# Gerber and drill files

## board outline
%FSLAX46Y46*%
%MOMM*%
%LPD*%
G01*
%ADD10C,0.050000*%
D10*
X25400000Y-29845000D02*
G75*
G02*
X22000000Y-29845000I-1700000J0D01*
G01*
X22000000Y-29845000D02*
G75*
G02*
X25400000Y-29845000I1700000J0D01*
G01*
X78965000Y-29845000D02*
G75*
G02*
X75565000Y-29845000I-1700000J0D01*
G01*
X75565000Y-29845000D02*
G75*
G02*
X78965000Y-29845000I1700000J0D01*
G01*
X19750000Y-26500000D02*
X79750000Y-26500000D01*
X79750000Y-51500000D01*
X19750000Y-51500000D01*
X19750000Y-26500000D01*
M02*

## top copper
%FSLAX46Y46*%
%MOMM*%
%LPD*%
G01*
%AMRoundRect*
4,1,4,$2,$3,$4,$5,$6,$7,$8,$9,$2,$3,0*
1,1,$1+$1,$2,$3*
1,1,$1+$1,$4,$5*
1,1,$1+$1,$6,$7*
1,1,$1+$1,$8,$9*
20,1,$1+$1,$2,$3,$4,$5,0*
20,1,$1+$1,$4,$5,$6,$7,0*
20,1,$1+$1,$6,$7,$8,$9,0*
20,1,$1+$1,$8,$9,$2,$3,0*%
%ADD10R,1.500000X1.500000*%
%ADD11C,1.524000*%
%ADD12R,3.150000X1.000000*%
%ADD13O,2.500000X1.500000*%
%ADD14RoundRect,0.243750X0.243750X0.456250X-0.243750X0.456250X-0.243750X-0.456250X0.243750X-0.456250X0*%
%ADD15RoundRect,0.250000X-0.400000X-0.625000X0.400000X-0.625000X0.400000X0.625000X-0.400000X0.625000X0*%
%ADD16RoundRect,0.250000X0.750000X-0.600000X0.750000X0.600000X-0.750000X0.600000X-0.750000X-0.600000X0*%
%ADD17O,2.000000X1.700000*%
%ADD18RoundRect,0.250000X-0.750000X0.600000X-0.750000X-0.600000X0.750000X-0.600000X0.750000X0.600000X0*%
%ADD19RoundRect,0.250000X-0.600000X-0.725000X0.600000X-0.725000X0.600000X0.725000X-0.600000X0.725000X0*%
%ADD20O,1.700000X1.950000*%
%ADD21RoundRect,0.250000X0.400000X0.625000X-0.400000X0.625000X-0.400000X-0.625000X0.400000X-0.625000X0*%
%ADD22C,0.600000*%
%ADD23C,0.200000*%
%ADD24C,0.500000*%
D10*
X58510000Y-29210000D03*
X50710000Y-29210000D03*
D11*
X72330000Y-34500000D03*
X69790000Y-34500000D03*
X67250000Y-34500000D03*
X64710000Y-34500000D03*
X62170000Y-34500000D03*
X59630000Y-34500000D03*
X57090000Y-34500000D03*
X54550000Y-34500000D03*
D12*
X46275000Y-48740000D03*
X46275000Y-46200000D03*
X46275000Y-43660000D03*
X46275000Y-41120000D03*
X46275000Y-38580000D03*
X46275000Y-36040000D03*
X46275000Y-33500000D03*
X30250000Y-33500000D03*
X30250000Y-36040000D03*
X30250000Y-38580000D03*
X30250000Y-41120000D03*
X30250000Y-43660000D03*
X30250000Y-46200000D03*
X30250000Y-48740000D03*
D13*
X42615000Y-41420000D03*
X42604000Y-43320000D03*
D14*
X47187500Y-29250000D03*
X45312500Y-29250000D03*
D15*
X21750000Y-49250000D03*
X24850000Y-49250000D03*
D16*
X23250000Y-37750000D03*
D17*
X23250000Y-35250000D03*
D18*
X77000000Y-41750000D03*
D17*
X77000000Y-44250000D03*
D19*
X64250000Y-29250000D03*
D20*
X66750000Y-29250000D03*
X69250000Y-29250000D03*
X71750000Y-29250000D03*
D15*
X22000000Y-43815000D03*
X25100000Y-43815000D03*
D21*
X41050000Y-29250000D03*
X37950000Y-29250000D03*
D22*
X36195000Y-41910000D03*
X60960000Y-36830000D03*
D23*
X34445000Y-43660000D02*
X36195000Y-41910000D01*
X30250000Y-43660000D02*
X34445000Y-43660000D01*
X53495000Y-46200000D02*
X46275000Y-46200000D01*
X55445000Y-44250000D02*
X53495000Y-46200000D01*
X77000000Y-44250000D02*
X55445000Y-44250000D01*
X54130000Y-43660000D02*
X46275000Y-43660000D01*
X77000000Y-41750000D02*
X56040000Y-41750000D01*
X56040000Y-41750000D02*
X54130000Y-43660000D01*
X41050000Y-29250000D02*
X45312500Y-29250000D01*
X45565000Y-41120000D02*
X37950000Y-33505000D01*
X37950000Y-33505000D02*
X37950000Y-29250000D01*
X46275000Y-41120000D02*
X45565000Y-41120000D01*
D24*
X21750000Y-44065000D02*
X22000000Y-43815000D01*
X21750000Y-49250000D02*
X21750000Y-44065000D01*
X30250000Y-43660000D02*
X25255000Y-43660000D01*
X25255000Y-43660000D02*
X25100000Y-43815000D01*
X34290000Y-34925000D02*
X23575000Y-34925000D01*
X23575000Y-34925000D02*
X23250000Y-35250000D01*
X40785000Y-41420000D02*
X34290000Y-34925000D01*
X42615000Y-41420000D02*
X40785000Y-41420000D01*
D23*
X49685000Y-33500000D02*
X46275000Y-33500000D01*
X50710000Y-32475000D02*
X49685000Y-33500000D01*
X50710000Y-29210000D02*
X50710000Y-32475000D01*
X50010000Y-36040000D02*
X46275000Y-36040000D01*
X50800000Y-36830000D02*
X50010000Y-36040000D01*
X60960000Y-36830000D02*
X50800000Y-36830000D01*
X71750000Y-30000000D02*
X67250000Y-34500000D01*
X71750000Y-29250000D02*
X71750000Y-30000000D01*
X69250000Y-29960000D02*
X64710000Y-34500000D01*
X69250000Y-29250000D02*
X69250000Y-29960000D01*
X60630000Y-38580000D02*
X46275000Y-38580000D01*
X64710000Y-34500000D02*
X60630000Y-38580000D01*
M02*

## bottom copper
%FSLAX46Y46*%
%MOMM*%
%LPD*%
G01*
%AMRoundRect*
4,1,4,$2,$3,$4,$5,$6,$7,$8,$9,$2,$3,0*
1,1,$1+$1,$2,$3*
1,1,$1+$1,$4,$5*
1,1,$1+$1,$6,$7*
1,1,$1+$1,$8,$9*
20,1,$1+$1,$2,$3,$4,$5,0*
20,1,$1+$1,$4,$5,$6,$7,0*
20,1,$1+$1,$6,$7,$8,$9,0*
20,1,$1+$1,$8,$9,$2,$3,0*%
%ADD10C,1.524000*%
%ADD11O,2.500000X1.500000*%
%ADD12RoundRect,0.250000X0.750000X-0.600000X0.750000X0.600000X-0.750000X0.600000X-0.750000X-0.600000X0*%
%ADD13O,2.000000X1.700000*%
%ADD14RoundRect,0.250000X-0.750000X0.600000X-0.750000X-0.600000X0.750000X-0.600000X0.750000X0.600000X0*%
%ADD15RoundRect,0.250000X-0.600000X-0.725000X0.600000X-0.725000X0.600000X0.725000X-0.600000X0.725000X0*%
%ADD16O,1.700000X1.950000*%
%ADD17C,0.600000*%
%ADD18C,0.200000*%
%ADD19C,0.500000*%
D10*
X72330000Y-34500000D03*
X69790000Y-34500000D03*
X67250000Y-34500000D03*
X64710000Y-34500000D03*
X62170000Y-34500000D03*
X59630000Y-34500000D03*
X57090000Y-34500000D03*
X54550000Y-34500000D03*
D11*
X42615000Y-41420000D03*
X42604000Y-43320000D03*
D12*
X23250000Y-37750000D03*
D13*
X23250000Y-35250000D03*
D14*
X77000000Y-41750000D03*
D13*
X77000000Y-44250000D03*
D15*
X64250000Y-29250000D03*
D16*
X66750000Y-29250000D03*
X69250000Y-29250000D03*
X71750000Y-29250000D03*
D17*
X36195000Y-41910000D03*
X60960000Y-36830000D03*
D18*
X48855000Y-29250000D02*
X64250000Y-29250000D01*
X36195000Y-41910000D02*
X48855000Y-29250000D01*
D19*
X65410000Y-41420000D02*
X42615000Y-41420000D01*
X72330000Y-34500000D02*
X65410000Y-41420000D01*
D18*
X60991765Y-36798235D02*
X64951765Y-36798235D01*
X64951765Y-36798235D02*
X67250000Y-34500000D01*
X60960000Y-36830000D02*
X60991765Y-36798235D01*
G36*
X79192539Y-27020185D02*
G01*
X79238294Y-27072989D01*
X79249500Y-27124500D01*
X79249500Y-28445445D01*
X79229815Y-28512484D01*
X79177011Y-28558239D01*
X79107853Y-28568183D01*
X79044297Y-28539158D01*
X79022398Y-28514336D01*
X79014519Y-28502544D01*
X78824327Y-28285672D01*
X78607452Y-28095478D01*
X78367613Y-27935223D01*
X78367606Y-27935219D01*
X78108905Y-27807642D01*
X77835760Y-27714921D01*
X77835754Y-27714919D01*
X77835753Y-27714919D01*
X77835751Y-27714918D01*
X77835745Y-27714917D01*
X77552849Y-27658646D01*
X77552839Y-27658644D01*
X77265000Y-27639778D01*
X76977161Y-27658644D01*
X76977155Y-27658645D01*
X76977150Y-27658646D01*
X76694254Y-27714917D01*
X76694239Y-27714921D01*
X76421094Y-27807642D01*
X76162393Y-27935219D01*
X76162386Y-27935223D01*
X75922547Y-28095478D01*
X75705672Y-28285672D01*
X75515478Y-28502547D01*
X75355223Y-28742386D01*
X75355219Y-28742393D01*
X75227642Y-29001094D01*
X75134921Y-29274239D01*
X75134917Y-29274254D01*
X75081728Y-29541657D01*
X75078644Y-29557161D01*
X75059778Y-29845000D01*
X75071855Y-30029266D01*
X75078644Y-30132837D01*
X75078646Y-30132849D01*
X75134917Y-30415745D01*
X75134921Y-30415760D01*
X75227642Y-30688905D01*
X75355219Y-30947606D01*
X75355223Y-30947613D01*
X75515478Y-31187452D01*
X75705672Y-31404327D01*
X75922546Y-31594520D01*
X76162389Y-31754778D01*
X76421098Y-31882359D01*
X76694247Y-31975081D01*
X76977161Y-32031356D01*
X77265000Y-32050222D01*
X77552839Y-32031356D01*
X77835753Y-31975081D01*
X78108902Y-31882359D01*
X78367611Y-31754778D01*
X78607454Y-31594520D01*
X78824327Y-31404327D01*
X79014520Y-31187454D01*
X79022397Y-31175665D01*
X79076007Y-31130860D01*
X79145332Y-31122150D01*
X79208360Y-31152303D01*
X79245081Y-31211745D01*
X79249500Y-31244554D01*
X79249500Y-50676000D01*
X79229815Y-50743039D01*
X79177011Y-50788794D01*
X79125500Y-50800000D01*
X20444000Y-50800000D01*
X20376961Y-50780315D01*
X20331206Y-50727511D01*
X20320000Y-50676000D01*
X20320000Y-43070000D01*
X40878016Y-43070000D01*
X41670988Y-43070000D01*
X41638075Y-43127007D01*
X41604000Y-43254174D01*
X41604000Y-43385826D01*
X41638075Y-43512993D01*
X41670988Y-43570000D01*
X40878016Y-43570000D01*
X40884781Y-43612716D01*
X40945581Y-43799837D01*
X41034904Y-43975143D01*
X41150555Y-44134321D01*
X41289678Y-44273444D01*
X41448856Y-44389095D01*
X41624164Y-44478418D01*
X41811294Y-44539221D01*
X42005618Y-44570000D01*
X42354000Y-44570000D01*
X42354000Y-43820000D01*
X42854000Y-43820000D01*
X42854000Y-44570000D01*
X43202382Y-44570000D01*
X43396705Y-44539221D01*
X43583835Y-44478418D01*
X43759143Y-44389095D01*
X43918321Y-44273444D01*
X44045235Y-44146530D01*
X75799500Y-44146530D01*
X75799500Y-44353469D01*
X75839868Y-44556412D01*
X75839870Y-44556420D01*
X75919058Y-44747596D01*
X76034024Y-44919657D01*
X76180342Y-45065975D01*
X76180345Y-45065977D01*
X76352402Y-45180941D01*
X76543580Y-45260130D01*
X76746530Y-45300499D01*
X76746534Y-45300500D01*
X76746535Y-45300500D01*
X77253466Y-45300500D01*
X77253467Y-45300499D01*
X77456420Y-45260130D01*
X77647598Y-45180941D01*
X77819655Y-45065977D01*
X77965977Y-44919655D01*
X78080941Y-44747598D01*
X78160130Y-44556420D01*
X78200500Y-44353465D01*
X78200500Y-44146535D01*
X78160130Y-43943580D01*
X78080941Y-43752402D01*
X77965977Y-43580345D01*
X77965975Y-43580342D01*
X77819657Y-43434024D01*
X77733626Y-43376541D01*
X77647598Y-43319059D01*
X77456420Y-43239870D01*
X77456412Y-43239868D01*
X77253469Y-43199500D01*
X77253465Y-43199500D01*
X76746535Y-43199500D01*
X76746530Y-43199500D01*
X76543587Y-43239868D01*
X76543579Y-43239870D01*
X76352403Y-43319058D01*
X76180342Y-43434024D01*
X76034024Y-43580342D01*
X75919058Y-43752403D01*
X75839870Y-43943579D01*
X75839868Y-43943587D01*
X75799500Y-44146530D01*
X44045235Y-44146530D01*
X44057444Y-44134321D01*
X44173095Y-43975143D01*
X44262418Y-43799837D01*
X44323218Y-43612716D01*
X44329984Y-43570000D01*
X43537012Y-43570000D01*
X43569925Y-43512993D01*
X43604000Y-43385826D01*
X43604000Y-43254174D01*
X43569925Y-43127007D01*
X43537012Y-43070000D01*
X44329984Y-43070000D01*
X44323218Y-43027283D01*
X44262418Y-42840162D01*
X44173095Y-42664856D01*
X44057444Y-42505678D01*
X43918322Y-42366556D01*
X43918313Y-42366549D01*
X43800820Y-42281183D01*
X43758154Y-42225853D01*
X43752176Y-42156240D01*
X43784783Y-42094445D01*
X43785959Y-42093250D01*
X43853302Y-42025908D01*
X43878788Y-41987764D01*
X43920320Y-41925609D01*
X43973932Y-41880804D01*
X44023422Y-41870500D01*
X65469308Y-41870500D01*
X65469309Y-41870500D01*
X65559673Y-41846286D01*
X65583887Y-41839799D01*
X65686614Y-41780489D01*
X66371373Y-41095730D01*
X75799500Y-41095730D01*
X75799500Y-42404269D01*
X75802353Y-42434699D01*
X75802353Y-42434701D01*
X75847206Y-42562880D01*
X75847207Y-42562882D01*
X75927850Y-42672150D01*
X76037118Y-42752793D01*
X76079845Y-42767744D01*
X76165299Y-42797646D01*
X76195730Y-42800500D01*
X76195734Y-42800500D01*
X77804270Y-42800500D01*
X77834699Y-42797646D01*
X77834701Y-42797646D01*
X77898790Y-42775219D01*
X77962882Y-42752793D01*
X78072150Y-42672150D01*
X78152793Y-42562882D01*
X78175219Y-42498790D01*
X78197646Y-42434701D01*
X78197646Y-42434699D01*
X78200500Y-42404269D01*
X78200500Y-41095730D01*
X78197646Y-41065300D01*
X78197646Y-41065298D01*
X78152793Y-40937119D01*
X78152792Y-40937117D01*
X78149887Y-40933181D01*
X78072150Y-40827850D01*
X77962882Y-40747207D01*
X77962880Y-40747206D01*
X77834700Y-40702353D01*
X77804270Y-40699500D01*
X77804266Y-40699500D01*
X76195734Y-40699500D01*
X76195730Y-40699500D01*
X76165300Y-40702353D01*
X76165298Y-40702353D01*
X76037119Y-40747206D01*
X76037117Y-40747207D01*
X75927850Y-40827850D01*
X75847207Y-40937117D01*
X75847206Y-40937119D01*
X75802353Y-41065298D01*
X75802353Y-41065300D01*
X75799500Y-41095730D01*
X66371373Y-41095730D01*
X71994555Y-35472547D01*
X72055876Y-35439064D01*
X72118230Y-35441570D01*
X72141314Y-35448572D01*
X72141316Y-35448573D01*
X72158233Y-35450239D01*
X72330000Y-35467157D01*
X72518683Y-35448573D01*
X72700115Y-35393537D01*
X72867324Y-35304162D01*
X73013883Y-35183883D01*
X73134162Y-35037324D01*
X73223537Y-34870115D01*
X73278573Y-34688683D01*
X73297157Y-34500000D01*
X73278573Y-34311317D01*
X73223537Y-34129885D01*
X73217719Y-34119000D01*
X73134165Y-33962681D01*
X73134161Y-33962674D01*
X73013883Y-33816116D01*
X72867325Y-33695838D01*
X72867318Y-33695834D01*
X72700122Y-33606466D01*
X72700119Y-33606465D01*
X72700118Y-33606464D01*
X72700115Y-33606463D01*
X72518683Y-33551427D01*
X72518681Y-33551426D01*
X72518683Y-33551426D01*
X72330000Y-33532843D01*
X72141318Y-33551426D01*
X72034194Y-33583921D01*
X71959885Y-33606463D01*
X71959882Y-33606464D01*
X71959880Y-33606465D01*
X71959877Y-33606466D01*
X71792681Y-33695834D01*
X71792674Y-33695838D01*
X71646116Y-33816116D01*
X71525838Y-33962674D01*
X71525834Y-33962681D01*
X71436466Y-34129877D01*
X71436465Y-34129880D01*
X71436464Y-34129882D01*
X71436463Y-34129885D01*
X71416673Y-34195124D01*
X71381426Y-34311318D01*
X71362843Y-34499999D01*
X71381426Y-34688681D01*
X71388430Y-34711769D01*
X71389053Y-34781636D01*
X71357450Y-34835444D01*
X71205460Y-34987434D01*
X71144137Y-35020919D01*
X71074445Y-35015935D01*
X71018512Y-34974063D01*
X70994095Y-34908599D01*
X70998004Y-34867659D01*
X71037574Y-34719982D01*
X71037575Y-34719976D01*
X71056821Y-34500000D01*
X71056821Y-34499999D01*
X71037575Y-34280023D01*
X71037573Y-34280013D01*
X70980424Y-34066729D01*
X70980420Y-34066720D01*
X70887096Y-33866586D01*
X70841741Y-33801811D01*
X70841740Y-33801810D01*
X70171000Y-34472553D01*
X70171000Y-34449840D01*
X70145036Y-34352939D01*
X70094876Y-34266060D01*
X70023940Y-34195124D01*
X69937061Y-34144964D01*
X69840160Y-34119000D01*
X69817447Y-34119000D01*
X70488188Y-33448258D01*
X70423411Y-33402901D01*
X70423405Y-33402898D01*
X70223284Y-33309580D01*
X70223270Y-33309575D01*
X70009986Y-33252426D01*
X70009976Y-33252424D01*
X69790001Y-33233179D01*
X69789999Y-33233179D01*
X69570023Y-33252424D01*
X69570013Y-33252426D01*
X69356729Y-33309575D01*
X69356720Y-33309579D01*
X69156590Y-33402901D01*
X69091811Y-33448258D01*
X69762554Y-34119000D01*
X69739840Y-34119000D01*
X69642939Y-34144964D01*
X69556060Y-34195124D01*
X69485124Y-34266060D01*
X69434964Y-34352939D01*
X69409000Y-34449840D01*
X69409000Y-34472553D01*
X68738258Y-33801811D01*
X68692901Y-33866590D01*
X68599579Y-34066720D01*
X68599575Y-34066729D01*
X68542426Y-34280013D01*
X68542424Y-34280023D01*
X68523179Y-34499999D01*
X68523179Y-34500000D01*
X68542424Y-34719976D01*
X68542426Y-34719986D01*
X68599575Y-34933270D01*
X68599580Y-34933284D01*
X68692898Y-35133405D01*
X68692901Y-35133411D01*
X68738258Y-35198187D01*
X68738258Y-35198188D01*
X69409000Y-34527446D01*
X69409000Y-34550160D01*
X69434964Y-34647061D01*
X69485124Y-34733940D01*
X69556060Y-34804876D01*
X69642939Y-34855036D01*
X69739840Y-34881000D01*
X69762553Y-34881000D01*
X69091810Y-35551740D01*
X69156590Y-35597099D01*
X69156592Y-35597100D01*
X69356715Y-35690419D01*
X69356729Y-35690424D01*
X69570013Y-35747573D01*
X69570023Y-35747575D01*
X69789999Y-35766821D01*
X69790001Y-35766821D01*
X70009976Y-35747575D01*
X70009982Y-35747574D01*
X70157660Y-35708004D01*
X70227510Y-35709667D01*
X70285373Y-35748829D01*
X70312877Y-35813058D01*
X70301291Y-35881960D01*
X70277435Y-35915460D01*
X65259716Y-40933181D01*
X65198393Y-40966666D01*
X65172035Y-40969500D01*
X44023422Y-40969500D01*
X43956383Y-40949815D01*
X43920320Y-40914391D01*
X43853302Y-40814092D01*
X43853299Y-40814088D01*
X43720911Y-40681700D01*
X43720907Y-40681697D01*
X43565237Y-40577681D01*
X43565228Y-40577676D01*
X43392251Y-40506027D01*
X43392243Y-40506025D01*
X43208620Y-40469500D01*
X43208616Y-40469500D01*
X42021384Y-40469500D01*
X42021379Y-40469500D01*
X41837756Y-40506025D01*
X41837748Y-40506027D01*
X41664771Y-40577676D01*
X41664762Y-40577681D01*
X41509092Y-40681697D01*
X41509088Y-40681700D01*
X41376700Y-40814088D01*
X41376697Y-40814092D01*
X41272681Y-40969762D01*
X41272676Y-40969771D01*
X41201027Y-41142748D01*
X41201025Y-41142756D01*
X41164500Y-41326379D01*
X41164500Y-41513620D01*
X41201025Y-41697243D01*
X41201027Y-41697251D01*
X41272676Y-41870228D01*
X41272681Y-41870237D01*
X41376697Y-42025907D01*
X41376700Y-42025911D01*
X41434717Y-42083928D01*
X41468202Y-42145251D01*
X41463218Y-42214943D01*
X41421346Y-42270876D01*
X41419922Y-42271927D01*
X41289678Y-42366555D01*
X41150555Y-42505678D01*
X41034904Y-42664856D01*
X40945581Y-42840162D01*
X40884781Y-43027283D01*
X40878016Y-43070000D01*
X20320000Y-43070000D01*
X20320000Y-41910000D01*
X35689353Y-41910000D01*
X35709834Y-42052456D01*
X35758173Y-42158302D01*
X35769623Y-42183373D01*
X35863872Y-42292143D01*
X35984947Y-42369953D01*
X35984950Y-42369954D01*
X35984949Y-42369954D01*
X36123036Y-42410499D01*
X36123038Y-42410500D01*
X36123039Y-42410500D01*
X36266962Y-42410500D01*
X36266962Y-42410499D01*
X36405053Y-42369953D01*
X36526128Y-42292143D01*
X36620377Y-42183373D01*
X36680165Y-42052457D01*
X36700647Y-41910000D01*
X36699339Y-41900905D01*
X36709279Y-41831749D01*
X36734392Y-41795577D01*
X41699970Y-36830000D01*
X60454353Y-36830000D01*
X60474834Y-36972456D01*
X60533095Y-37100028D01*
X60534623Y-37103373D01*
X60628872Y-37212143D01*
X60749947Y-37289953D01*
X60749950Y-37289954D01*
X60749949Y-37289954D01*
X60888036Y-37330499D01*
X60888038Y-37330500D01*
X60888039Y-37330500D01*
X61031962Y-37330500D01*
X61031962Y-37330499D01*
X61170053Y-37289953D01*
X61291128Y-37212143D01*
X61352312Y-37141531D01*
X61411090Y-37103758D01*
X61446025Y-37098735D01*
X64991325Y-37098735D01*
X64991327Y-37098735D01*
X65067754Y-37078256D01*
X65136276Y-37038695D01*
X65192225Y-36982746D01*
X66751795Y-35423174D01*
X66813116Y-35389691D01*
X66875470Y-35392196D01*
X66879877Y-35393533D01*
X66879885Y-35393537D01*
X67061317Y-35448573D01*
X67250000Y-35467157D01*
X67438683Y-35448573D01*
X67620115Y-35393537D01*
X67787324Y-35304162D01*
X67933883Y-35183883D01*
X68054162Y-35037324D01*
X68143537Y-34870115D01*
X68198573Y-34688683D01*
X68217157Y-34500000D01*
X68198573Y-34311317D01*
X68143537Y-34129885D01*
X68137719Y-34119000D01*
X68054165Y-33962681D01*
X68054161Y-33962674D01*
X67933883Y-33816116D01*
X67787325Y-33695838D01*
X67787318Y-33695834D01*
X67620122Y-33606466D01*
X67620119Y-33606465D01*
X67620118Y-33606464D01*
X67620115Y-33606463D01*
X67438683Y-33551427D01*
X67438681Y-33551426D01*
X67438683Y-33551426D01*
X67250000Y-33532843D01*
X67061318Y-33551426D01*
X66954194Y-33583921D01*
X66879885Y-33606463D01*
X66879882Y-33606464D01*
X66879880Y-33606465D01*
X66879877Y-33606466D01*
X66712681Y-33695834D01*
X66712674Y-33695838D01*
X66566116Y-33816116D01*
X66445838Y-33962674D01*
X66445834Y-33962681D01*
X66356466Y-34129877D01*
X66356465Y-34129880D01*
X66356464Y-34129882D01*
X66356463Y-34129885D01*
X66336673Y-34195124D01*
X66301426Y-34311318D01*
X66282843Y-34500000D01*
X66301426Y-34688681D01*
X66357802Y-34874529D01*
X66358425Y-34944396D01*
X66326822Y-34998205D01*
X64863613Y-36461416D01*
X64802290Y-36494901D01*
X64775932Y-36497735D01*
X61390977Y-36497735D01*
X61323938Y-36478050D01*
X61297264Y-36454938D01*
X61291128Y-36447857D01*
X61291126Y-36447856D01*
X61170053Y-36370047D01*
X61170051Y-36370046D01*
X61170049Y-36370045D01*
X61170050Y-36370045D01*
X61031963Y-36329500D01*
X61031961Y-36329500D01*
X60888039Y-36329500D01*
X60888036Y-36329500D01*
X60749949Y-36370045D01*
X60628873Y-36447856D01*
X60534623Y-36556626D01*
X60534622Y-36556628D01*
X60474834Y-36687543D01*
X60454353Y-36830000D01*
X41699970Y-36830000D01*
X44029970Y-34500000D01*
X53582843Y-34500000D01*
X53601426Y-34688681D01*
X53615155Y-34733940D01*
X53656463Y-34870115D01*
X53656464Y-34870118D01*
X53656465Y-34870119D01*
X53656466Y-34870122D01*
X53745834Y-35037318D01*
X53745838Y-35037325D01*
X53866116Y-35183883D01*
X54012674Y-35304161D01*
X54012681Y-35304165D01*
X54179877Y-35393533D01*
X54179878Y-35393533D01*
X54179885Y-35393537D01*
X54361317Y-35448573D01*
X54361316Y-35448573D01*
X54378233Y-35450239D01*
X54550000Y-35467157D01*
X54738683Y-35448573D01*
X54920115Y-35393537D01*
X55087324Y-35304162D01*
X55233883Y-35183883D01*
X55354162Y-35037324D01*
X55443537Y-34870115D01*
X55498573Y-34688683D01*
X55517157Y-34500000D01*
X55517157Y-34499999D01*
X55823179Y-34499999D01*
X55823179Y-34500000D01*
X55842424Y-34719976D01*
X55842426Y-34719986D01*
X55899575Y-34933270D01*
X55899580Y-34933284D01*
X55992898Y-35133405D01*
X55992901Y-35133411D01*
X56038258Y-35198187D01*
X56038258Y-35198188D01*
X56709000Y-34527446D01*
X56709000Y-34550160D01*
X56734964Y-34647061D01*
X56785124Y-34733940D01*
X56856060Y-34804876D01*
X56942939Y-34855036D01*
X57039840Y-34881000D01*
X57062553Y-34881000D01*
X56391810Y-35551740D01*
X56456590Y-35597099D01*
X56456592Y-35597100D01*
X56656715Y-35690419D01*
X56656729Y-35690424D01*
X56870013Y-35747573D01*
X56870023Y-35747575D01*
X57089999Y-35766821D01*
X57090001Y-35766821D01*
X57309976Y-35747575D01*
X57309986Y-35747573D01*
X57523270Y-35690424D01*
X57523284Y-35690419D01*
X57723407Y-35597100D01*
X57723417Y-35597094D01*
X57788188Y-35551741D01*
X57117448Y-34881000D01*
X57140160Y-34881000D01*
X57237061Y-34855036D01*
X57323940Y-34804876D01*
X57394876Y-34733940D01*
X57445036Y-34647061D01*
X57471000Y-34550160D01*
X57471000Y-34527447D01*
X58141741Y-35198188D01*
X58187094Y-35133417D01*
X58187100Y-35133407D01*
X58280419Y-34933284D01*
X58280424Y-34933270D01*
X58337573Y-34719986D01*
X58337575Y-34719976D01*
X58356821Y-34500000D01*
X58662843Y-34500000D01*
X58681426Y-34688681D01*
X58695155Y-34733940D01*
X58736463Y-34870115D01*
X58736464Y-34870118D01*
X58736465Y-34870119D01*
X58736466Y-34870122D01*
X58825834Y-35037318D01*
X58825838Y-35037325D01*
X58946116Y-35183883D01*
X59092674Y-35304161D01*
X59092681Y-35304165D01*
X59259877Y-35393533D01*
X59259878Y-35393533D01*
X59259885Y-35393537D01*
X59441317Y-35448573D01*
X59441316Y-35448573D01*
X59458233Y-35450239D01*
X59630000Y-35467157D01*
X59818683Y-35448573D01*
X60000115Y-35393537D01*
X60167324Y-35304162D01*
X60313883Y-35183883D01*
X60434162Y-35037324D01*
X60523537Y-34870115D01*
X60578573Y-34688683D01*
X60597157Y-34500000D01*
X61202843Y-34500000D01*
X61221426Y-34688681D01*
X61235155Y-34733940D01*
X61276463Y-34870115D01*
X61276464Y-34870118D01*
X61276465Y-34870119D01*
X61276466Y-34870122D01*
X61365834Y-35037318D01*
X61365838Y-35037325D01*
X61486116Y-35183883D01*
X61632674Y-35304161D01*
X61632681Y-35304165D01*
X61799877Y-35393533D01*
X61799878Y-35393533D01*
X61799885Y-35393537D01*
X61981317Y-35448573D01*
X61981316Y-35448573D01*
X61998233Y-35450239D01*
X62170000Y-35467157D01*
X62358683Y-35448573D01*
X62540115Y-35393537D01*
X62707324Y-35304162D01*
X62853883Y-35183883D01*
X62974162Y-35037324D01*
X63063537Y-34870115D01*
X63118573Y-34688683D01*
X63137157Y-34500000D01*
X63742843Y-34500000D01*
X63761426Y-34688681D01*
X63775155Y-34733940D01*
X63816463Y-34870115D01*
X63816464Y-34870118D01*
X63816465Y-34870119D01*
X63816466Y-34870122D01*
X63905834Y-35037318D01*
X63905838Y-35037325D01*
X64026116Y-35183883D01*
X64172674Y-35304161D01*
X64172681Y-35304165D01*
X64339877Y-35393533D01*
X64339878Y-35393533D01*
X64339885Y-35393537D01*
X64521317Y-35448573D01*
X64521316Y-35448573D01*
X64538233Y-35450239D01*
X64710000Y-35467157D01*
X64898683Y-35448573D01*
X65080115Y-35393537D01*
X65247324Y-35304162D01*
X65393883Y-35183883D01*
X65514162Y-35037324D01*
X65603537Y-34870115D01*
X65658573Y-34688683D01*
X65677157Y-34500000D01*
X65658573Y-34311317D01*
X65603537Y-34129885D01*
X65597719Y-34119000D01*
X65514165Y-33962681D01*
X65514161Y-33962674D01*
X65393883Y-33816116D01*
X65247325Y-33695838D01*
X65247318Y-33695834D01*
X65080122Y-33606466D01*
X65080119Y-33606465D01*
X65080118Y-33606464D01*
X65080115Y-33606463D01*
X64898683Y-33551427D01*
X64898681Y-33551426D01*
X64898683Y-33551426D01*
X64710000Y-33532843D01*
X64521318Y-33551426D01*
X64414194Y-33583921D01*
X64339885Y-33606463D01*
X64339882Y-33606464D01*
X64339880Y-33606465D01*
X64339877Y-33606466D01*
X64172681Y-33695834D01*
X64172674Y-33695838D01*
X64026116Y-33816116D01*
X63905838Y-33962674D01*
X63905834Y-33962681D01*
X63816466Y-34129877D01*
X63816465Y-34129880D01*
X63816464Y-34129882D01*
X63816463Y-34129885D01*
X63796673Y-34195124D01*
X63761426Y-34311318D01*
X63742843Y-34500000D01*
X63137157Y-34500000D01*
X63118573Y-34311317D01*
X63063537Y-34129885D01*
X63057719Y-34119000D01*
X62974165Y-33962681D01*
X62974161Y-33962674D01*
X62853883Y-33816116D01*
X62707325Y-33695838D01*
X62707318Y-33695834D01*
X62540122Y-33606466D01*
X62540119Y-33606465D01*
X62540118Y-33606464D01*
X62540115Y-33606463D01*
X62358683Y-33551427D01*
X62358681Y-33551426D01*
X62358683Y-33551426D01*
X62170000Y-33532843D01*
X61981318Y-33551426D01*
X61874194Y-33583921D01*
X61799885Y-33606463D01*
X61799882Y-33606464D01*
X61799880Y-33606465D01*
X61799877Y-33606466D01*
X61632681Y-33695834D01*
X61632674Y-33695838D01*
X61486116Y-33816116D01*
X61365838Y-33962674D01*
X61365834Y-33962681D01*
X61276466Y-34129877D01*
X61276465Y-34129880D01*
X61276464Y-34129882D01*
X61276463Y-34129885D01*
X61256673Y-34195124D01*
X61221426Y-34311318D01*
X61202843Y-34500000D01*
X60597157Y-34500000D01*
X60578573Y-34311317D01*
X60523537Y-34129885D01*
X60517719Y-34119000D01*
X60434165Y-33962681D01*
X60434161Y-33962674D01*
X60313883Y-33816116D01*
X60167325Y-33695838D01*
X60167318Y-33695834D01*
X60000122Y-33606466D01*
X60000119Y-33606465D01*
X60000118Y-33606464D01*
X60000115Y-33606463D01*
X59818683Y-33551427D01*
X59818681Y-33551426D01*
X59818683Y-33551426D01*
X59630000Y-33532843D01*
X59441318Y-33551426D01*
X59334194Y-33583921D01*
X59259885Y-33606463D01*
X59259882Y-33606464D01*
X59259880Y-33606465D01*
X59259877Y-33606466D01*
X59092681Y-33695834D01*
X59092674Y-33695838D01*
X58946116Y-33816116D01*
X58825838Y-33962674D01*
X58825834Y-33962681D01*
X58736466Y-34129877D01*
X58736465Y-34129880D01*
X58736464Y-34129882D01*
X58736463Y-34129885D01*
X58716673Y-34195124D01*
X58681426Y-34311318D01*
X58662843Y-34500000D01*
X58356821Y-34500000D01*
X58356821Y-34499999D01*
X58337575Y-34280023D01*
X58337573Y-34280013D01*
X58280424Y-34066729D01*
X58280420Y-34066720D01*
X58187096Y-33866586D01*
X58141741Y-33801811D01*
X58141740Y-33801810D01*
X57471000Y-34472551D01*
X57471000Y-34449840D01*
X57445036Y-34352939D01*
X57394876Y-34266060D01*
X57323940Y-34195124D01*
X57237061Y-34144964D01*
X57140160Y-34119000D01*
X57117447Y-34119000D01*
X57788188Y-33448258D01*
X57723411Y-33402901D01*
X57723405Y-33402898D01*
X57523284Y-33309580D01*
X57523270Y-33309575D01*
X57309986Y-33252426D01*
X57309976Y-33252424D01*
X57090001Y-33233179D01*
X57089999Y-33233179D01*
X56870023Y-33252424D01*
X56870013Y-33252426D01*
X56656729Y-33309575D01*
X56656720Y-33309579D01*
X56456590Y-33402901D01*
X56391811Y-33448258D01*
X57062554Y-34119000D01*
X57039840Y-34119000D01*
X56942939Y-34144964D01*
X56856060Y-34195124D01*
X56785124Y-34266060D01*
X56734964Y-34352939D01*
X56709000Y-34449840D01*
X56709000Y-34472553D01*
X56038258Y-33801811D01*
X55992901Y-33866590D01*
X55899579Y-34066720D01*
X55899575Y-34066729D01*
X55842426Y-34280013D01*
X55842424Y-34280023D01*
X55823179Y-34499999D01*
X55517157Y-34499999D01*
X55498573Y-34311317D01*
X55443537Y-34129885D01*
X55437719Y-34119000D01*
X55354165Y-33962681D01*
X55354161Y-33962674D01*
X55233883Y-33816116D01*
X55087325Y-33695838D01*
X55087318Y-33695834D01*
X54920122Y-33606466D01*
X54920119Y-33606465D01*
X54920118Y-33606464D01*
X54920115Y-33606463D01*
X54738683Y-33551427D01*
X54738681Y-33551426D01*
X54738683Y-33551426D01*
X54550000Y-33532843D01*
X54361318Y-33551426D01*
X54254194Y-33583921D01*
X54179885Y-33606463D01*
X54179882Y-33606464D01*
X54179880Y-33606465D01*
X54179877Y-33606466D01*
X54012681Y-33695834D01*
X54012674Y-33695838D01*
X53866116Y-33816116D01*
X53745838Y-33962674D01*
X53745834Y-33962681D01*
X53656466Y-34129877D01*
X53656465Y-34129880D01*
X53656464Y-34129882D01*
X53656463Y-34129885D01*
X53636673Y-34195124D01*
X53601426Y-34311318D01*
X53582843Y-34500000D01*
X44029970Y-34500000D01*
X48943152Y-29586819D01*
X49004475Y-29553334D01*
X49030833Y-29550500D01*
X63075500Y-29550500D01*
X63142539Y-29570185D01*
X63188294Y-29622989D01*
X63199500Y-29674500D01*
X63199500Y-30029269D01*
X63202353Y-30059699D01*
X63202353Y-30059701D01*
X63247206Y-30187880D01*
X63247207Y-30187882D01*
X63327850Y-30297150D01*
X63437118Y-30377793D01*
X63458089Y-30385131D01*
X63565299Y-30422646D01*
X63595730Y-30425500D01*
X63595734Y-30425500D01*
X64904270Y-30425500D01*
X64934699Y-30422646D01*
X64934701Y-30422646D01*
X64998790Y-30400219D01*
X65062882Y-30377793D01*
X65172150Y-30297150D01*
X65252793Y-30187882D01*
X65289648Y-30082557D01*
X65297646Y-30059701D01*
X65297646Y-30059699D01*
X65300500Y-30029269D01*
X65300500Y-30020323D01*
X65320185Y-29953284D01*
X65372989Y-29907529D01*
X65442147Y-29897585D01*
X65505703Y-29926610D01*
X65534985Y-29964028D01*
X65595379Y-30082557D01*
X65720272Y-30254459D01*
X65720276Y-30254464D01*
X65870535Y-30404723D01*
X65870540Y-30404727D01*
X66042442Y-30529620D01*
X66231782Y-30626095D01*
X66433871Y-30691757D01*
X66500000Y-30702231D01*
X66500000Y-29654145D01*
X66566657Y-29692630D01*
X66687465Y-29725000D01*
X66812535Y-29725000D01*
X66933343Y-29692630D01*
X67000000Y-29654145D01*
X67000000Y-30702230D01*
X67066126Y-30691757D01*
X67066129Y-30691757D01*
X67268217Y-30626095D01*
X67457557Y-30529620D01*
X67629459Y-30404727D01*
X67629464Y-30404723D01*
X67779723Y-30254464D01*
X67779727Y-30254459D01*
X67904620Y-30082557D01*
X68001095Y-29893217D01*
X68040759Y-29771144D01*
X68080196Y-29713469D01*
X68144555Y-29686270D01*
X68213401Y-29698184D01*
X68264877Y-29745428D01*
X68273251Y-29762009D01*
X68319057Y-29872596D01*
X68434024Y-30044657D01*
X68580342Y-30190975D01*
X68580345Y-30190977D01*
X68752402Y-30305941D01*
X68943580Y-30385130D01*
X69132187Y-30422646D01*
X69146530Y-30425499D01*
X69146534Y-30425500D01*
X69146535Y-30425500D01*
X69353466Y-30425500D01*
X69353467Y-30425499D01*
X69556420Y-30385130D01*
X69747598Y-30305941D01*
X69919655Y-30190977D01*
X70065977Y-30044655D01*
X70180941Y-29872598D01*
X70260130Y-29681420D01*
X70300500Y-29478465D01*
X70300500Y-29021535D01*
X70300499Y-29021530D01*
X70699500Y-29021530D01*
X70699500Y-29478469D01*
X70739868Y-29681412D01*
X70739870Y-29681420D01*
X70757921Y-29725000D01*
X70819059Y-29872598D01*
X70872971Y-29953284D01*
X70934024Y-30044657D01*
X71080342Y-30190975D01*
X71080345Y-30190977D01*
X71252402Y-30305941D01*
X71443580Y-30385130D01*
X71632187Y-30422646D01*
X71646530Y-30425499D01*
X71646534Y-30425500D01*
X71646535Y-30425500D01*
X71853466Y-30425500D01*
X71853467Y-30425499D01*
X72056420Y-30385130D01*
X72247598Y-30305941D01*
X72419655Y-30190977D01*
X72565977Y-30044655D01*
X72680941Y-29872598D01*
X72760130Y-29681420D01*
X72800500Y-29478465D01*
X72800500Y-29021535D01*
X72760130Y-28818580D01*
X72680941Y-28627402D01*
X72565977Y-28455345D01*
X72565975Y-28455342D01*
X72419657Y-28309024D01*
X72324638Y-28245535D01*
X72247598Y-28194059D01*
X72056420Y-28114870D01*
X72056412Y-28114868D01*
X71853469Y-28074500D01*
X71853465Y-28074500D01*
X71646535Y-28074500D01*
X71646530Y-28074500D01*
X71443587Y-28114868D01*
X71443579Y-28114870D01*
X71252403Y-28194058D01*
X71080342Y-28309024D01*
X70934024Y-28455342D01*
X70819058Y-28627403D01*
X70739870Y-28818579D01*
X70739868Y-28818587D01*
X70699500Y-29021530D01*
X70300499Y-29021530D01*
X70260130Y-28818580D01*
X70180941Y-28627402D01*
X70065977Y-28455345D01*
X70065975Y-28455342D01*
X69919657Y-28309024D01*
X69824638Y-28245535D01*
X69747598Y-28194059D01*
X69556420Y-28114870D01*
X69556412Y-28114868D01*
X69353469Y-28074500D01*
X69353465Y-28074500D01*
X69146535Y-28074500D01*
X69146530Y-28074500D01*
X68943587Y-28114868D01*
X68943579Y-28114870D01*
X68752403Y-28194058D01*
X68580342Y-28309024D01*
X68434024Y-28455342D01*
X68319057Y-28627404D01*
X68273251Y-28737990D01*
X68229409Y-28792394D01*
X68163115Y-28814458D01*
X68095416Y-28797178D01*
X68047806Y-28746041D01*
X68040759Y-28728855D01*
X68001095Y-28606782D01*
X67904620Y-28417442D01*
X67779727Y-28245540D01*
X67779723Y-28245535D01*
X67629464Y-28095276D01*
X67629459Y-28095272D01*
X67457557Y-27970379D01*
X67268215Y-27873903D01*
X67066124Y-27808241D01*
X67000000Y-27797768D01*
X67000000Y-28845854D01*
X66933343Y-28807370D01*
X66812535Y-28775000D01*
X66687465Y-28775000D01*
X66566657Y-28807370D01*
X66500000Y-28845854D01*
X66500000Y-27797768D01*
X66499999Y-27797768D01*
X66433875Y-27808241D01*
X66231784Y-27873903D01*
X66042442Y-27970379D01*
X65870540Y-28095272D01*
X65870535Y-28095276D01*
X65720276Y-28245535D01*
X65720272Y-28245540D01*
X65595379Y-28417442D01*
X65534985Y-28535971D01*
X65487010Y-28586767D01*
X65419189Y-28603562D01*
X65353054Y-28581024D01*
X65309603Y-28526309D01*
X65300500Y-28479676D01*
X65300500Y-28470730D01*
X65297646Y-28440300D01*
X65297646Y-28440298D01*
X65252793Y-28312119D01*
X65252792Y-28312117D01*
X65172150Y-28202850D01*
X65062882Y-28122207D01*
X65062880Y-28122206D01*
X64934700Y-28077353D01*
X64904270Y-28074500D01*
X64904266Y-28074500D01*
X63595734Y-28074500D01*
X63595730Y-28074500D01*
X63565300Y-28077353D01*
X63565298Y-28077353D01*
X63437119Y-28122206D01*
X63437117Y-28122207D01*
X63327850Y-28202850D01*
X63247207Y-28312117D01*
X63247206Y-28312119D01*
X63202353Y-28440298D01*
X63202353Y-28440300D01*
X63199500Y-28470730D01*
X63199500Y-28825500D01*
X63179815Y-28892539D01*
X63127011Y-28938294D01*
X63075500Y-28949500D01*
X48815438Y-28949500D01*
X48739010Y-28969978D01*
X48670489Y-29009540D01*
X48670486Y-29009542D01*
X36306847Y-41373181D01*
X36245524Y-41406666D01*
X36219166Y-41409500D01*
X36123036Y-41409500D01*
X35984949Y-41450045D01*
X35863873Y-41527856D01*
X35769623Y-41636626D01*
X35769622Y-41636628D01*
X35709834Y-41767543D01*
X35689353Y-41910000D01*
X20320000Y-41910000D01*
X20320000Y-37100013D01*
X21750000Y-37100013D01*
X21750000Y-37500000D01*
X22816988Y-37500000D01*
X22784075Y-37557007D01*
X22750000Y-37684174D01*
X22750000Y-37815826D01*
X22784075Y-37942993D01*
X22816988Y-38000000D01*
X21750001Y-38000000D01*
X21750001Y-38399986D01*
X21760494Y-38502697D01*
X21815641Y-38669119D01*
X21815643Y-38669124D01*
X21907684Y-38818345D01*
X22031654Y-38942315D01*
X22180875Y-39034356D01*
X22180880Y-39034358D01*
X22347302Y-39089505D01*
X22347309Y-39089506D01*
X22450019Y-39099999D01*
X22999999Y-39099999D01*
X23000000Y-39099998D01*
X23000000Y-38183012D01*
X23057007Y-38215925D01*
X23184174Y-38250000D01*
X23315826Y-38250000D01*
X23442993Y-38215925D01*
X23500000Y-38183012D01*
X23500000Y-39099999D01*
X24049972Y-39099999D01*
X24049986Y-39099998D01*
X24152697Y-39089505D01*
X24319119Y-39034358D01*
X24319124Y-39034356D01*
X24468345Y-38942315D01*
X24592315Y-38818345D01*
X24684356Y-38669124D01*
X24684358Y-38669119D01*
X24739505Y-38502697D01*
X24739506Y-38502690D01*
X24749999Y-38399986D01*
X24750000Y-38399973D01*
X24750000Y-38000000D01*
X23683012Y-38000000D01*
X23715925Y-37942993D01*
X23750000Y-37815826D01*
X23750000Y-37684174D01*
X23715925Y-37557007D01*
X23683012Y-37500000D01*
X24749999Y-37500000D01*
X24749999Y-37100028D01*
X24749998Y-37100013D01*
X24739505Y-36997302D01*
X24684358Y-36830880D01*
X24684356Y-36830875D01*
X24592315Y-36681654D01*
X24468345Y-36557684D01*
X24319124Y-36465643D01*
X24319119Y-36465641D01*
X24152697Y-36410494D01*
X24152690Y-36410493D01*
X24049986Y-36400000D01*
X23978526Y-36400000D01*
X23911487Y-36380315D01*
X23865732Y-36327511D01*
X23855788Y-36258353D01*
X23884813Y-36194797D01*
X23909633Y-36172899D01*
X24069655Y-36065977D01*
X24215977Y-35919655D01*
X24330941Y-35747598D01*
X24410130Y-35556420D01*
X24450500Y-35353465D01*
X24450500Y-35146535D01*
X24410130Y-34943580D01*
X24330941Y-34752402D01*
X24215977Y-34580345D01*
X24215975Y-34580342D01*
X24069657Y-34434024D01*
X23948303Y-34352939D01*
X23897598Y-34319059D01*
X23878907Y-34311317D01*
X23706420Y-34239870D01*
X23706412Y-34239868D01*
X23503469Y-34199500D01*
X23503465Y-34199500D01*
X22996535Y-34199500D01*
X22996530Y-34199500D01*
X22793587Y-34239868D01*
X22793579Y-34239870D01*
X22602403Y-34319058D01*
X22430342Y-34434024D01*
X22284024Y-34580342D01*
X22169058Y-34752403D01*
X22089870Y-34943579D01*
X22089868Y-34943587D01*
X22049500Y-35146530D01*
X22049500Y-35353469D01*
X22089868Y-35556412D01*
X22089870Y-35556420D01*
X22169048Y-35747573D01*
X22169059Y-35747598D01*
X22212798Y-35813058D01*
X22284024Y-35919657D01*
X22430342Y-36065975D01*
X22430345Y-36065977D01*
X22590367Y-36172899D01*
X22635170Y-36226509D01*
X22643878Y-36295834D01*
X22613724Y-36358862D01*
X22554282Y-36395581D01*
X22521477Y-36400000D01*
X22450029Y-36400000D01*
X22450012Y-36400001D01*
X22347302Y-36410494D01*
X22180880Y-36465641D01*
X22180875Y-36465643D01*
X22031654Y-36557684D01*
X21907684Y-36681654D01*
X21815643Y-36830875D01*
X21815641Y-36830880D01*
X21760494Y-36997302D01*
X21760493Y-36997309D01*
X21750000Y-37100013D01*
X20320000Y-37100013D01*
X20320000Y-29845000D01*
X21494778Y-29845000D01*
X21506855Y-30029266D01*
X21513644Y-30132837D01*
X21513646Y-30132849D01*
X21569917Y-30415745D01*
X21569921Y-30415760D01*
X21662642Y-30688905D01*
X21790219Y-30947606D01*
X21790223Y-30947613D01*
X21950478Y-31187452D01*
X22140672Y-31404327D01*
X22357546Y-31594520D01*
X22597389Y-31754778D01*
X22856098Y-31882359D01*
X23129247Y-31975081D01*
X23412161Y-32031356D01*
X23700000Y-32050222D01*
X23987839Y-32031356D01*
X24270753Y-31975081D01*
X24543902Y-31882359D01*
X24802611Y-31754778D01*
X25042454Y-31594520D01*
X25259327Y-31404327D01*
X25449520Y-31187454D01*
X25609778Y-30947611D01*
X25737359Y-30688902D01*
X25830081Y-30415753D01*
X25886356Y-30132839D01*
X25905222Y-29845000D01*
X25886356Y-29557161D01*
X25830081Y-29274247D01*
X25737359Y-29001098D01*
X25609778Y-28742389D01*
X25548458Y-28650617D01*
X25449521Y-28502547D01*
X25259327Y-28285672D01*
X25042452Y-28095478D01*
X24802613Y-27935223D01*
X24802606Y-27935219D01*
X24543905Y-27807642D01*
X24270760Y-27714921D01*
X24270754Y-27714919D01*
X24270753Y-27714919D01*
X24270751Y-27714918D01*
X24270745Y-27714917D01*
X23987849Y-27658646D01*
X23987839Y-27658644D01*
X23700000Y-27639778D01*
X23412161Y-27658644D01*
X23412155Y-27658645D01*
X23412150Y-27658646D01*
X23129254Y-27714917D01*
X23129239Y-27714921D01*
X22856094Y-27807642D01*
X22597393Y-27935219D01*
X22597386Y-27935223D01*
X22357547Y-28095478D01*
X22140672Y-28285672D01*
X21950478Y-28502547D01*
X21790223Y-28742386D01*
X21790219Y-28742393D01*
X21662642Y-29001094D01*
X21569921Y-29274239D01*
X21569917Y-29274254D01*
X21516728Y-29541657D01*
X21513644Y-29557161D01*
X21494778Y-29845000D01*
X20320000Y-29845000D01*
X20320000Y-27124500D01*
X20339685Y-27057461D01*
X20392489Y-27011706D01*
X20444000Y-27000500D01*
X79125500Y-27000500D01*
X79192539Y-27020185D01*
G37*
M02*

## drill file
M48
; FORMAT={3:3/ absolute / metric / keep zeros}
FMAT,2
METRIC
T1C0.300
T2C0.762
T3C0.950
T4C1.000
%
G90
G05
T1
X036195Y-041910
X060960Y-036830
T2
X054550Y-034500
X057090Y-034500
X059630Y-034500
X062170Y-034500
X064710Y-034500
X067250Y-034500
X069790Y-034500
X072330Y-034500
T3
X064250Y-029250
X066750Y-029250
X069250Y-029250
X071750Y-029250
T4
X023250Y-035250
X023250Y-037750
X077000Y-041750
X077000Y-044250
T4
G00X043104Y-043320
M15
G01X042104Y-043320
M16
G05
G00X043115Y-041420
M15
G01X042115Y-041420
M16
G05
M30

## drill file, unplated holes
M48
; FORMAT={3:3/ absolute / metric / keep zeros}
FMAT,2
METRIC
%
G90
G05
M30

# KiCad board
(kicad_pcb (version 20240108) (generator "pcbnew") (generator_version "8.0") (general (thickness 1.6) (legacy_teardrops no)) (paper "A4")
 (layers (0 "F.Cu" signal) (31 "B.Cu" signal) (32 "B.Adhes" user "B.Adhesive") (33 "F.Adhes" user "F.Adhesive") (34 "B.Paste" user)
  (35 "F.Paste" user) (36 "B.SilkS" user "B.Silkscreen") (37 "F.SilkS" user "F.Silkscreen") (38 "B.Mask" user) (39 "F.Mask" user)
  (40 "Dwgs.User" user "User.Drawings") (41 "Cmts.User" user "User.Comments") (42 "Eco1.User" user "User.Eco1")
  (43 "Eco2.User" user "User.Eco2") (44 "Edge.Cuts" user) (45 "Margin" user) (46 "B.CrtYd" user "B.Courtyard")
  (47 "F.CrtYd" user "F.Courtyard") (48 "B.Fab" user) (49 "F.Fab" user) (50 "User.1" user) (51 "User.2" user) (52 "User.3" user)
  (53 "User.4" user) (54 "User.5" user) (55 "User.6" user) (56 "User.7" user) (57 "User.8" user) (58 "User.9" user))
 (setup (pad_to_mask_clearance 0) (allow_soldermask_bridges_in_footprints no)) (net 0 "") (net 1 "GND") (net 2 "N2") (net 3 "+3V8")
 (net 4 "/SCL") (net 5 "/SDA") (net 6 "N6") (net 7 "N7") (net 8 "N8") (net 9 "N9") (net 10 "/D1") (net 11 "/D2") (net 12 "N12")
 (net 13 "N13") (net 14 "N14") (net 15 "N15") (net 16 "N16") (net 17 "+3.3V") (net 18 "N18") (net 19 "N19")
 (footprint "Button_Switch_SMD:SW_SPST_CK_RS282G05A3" (layer "F.Cu") (at 54.61 29.21 180)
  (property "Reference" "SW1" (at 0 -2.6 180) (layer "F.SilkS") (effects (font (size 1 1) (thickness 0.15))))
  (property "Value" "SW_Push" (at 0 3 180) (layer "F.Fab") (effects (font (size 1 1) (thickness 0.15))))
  (pad "1" smd rect (at -3.9 0 180) (size 1.5 1.5) (layers "F.Cu" "F.Paste" "F.Mask") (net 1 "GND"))
  (pad "2" smd rect (at 3.9 0 180) (size 1.5 1.5) (layers "F.Cu" "F.Paste" "F.Mask") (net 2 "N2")))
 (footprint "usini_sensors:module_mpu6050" (layer "F.Cu") (at 54.55 34.5 -90)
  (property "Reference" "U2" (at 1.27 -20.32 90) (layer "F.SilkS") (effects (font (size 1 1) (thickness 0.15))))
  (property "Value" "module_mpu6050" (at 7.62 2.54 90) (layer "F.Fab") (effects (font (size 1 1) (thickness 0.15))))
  (pad "1" thru_hole circle (at 0 -17.78 270) (size 1.524 1.524) (drill 0.762) (layers "*.Cu" "*.Mask") (remove_unused_layers no)
   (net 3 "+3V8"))
  (pad "2" thru_hole circle (at 0 -15.24 270) (size 1.524 1.524) (drill 0.762) (layers "*.Cu" "*.Mask") (remove_unused_layers no)
   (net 1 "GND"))
  (pad "3" thru_hole circle (at 0 -12.7 270) (size 1.524 1.524) (drill 0.762) (layers "*.Cu" "*.Mask") (remove_unused_layers no)
   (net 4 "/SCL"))
  (pad "4" thru_hole circle (at 0 -10.16 270) (size 1.524 1.524) (drill 0.762) (layers "*.Cu" "*.Mask") (remove_unused_layers no)
   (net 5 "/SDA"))
  (pad "5" thru_hole circle (at 0 -7.62 270) (size 1.524 1.524) (drill 0.762) (layers "*.Cu" "*.Mask") (remove_unused_layers no)
   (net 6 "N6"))
  (pad "6" thru_hole circle (at 0 -5.08 270) (size 1.524 1.524) (drill 0.762) (layers "*.Cu" "*.Mask") (remove_unused_layers no)
   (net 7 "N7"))
  (pad "7" thru_hole circle (at 0 -2.54 270) (size 1.524 1.524) (drill 0.762) (layers "*.Cu" "*.Mask") (remove_unused_layers no)
   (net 1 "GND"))
  (pad "8" thru_hole circle (at 0 0 270) (size 1.524 1.524) (drill 0.762) (layers "*.Cu" "*.Mask") (remove_unused_layers no) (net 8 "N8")))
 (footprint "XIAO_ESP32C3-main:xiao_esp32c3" (layer "F.Cu") (at 37.675 39.32 180)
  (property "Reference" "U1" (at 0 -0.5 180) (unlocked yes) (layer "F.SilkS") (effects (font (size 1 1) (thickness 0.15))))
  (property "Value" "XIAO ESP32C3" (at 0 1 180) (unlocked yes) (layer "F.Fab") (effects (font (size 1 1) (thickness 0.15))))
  (pad "1" smd rect (at -8.6 -9.42 180) (size 3.15 1) (layers "F.Cu" "F.Paste" "F.Mask") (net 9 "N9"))
  (pad "2" smd rect (at -8.6 -6.88 180) (size 3.15 1) (layers "F.Cu" "F.Paste" "F.Mask") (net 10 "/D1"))
  (pad "3" smd rect (at -8.6 -4.34 180) (size 3.15 1) (layers "F.Cu" "F.Paste" "F.Mask") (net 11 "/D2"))
  (pad "4" smd rect (at -8.6 -1.8 180) (size 3.15 1) (layers "F.Cu" "F.Paste" "F.Mask") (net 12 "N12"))
  (pad "5" smd rect (at -8.6 0.74 180) (size 3.15 1) (layers "F.Cu" "F.Paste" "F.Mask") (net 5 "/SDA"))
  (pad "6" smd rect (at -8.6 3.28 180) (size 3.15 1) (layers "F.Cu" "F.Paste" "F.Mask") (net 4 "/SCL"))
  (pad "7" smd rect (at -8.6 5.82 180) (size 3.15 1) (layers "F.Cu" "F.Paste" "F.Mask") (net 2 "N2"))
  (pad "8" smd rect (at 7.425 5.82 180) (size 3.15 1) (layers "F.Cu" "F.Paste" "F.Mask") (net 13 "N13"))
  (pad "9" smd rect (at 7.425 3.28 180) (size 3.15 1) (layers "F.Cu" "F.Paste" "F.Mask") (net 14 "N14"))
  (pad "10" smd rect (at 7.425 0.74 180) (size 3.15 1) (layers "F.Cu" "F.Paste" "F.Mask") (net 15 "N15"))
  (pad "11" smd rect (at 7.425 -1.8 180) (size 3.15 1) (layers "F.Cu" "F.Paste" "F.Mask") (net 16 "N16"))
  (pad "12" smd rect (at 7.425 -4.34 180) (size 3.15 1) (layers "F.Cu" "F.Paste" "F.Mask") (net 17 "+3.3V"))
  (pad "13" smd rect (at 7.425 -6.88 180) (size 3.15 1) (layers "F.Cu" "F.Paste" "F.Mask") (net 1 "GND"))
  (pad "14" smd rect (at 7.425 -9.42 180) (size 3.15 1) (layers "F.Cu" "F.Paste" "F.Mask") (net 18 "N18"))
  (pad "B+" thru_hole oval (at -4.94 -2.1 180) (size 2.5 1.5) (drill oval 2 1) (layers "*.Cu" "*.Mask") (remove_unused_layers no)
   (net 3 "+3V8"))
  (pad "B-" thru_hole oval (at -4.929 -4 180) (size 2.5 1.5) (drill oval 2 1) (layers "*.Cu" "*.Mask") (remove_unused_layers no)
   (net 1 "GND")))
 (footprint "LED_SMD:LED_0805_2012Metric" (layer "F.Cu") (at 46.25 29.25 180)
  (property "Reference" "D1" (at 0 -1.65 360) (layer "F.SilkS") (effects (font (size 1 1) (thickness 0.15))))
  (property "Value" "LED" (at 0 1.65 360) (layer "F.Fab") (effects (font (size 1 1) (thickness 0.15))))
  (pad "1" smd roundrect (at -0.9375 0 180) (size 0.975 1.4) (layers "F.Cu" "F.Paste" "F.Mask") (roundrect_rratio 0.25) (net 1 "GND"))
  (pad "2" smd roundrect (at 0.9375 0 180) (size 0.975 1.4) (layers "F.Cu" "F.Paste" "F.Mask") (roundrect_rratio 0.25) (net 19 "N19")))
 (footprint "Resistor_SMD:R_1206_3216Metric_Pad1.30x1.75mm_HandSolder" (layer "F.Cu") (at 23.3 49.25)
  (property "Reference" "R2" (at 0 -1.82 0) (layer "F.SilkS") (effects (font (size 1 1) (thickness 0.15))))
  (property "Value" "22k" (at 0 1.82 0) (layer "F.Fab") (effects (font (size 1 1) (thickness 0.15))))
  (pad "1" smd roundrect (at -1.55 0) (size 1.3 1.75) (layers "F.Cu" "F.Paste" "F.Mask") (roundrect_rratio 0.192308) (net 9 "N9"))
  (pad "2" smd roundrect (at 1.55 0) (size 1.3 1.75) (layers "F.Cu" "F.Paste" "F.Mask") (roundrect_rratio 0.192308) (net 1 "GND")))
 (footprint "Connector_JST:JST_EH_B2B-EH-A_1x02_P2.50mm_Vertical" (layer "F.Cu") (at 23.25 37.75 90)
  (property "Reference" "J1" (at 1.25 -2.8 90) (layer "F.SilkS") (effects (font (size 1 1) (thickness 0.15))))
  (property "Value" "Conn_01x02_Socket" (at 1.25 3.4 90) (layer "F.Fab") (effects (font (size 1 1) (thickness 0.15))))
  (pad "1" thru_hole roundrect (at 0 0 90) (size 1.7 2) (drill 1) (layers "*.Cu" "*.Mask") (remove_unused_layers no)
   (roundrect_rratio 0.147059) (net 1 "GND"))
  (pad "2" thru_hole oval (at 2.5 0 90) (size 1.7 2) (drill 1) (layers "*.Cu" "*.Mask") (remove_unused_layers no) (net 3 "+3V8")))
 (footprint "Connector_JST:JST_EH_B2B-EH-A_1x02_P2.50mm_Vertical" (layer "F.Cu") (at 77 41.75 -90)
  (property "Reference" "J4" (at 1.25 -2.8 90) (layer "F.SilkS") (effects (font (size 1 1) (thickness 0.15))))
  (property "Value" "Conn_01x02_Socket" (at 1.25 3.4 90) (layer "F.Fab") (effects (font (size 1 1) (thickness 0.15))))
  (pad "1" thru_hole roundrect (at 0 0 270) (size 1.7 2) (drill 1) (layers "*.Cu" "*.Mask") (remove_unused_layers no)
   (roundrect_rratio 0.147059) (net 11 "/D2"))
  (pad "2" thru_hole oval (at 2.5 0 270) (size 1.7 2) (drill 1) (layers "*.Cu" "*.Mask") (remove_unused_layers no) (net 10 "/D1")))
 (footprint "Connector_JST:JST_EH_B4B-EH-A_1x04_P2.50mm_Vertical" (layer "F.Cu") (at 64.25 29.25)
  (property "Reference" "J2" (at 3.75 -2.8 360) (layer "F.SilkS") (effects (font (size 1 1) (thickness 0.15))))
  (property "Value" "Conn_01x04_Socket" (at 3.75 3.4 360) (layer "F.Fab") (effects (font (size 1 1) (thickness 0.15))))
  (pad "1" thru_hole roundrect (at 0 0) (size 1.7 1.95) (drill 0.95) (layers "*.Cu" "*.Mask") (remove_unused_layers no)
   (roundrect_rratio 0.147059) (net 17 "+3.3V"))
  (pad "2" thru_hole oval (at 2.5 0) (size 1.7 1.95) (drill 0.95) (layers "*.Cu" "*.Mask") (remove_unused_layers no) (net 1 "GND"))
  (pad "3" thru_hole oval (at 5 0) (size 1.7 1.95) (drill 0.95) (layers "*.Cu" "*.Mask") (remove_unused_layers no) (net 5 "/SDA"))
  (pad "4" thru_hole oval (at 7.5 0) (size 1.7 1.95) (drill 0.95) (layers "*.Cu" "*.Mask") (remove_unused_layers no) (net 4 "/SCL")))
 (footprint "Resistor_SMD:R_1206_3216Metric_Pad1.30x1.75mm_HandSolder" (layer "F.Cu") (at 23.55 43.815)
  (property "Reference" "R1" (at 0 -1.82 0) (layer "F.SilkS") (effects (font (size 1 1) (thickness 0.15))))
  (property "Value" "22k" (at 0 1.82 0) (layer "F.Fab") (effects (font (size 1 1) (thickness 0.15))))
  (pad "1" smd roundrect (at -1.55 0) (size 1.3 1.75) (layers "F.Cu" "F.Paste" "F.Mask") (roundrect_rratio 0.192308) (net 9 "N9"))
  (pad "2" smd roundrect (at 1.55 0) (size 1.3 1.75) (layers "F.Cu" "F.Paste" "F.Mask") (roundrect_rratio 0.192308) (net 17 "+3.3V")))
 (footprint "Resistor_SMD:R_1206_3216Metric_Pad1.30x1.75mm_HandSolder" (layer "F.Cu") (at 39.5 29.25 180)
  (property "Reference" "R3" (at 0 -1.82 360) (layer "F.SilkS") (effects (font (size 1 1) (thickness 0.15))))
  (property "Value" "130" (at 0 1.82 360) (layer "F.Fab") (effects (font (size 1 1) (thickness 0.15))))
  (pad "1" smd roundrect (at -1.55 0 180) (size 1.3 1.75) (layers "F.Cu" "F.Paste" "F.Mask") (roundrect_rratio 0.192308) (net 19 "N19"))
  (pad "2" smd roundrect (at 1.55 0 180) (size 1.3 1.75) (layers "F.Cu" "F.Paste" "F.Mask") (roundrect_rratio 0.192308) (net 12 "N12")))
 (gr_circle (center 77.265 29.845) (end 78.965 29.845) (stroke (width 0.05) (type default)) (fill none) (layer "Edge.Cuts"))
 (gr_circle (center 23.7 29.845) (end 25.4 29.845) (stroke (width 0.05) (type default)) (fill none) (layer "Edge.Cuts"))
 (gr_rect (start 19.75 26.5) (end 79.75 51.5) (stroke (width 0.05) (type default)) (fill none) (layer "Edge.Cuts"))
 (segment (start 41.05 29.25) (end 45.3125 29.25) (width 0.2) (layer "F.Cu") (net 19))
 (segment (start 23.575 34.925) (end 23.25 35.25) (width 0.5) (layer "F.Cu") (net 3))
 (segment (start 34.29 34.925) (end 23.575 34.925) (width 0.5) (layer "F.Cu") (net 3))
 (segment (start 42.615 41.42) (end 40.785 41.42) (width 0.5) (layer "F.Cu") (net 3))
 (segment (start 40.785 41.42) (end 34.29 34.925) (width 0.5) (layer "F.Cu") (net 3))
 (segment (start 72.33 34.5) (end 65.41 41.42) (width 0.5) (layer "B.Cu") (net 3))
 (segment (start 65.41 41.42) (end 42.615 41.42) (width 0.5) (layer "B.Cu") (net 3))
 (segment (start 69.25 29.25) (end 69.25 29.96) (width 0.2) (layer "F.Cu") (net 5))
 (segment (start 69.25 29.96) (end 64.71 34.5) (width 0.2) (layer "F.Cu") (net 5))
 (segment (start 64.71 34.5) (end 60.63 38.58) (width 0.2) (layer "F.Cu") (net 5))
 (segment (start 60.63 38.58) (end 46.275 38.58) (width 0.2) (layer "F.Cu") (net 5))
 (segment (start 60.96 36.83) (end 50.8 36.83) (width 0.2) (layer "F.Cu") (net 4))
 (segment (start 50.8 36.83) (end 50.01 36.04) (width 0.2) (layer "F.Cu") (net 4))
 (segment (start 50.01 36.04) (end 46.275 36.04) (width 0.2) (layer "F.Cu") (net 4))
 (segment (start 71.75 30) (end 67.25 34.5) (width 0.2) (layer "F.Cu") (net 4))
 (segment (start 71.75 29.25) (end 71.75 30) (width 0.2) (layer "F.Cu") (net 4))
 (via (at 60.96 36.83) (size 0.6) (drill 0.3) (layers "F.Cu" "B.Cu") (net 4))
 (segment (start 64.951765 36.798235) (end 67.25 34.5) (width 0.2) (layer "B.Cu") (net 4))
 (segment (start 60.991765 36.798235) (end 64.951765 36.798235) (width 0.2) (layer "B.Cu") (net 4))
 (segment (start 60.96 36.83) (end 60.991765 36.798235) (width 0.2) (layer "B.Cu") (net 4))
 (segment (start 34.445 43.66) (end 36.195 41.91) (width 0.2) (layer "F.Cu") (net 17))
 (segment (start 30.25 43.66) (end 25.255 43.66) (width 0.5) (layer "F.Cu") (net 17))
 (segment (start 25.255 43.66) (end 25.1 43.815) (width 0.5) (layer "F.Cu") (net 17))
 (segment (start 30.25 43.66) (end 34.445 43.66) (width 0.2) (layer "F.Cu") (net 17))
 (via (at 36.195 41.91) (size 0.6) (drill 0.3) (layers "F.Cu" "B.Cu") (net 17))
 (segment (start 36.195 41.91) (end 48.855 29.25) (width 0.2) (layer "B.Cu") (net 17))
 (segment (start 48.855 29.25) (end 64.25 29.25) (width 0.2) (layer "B.Cu") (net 17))
 (segment (start 54.13 43.66) (end 46.275 43.66) (width 0.2) (layer "F.Cu") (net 11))
 (segment (start 77 41.75) (end 56.04 41.75) (width 0.2) (layer "F.Cu") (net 11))
 (segment (start 56.04 41.75) (end 54.13 43.66) (width 0.2) (layer "F.Cu") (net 11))
 (segment (start 77 44.25) (end 55.445 44.25) (width 0.2) (layer "F.Cu") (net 10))
 (segment (start 53.495 46.2) (end 46.275 46.2) (width 0.2) (layer "F.Cu") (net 10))
 (segment (start 55.445 44.25) (end 53.495 46.2) (width 0.2) (layer "F.Cu") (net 10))
 (segment (start 21.75 49.25) (end 21.75 44.065) (width 0.5) (layer "F.Cu") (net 9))
 (segment (start 21.75 44.065) (end 22 43.815) (width 0.5) (layer "F.Cu") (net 9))
 (segment (start 46.275 41.12) (end 45.565 41.12) (width 0.2) (layer "F.Cu") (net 12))
 (segment (start 45.565 41.12) (end 37.95 33.505) (width 0.2) (layer "F.Cu") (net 12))
 (segment (start 37.95 33.505) (end 37.95 29.25) (width 0.2) (layer "F.Cu") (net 12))
 (segment (start 50.71 32.475) (end 49.685 33.5) (width 0.2) (layer "F.Cu") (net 2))
 (segment (start 50.71 29.21) (end 50.71 32.475) (width 0.2) (layer "F.Cu") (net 2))
 (segment (start 49.685 33.5) (end 46.275 33.5) (width 0.2) (layer "F.Cu") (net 2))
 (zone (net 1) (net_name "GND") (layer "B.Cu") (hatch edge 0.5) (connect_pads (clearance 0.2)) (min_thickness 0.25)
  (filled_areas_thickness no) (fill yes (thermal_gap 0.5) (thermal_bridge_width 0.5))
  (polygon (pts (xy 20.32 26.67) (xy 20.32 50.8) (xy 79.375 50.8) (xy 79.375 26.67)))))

